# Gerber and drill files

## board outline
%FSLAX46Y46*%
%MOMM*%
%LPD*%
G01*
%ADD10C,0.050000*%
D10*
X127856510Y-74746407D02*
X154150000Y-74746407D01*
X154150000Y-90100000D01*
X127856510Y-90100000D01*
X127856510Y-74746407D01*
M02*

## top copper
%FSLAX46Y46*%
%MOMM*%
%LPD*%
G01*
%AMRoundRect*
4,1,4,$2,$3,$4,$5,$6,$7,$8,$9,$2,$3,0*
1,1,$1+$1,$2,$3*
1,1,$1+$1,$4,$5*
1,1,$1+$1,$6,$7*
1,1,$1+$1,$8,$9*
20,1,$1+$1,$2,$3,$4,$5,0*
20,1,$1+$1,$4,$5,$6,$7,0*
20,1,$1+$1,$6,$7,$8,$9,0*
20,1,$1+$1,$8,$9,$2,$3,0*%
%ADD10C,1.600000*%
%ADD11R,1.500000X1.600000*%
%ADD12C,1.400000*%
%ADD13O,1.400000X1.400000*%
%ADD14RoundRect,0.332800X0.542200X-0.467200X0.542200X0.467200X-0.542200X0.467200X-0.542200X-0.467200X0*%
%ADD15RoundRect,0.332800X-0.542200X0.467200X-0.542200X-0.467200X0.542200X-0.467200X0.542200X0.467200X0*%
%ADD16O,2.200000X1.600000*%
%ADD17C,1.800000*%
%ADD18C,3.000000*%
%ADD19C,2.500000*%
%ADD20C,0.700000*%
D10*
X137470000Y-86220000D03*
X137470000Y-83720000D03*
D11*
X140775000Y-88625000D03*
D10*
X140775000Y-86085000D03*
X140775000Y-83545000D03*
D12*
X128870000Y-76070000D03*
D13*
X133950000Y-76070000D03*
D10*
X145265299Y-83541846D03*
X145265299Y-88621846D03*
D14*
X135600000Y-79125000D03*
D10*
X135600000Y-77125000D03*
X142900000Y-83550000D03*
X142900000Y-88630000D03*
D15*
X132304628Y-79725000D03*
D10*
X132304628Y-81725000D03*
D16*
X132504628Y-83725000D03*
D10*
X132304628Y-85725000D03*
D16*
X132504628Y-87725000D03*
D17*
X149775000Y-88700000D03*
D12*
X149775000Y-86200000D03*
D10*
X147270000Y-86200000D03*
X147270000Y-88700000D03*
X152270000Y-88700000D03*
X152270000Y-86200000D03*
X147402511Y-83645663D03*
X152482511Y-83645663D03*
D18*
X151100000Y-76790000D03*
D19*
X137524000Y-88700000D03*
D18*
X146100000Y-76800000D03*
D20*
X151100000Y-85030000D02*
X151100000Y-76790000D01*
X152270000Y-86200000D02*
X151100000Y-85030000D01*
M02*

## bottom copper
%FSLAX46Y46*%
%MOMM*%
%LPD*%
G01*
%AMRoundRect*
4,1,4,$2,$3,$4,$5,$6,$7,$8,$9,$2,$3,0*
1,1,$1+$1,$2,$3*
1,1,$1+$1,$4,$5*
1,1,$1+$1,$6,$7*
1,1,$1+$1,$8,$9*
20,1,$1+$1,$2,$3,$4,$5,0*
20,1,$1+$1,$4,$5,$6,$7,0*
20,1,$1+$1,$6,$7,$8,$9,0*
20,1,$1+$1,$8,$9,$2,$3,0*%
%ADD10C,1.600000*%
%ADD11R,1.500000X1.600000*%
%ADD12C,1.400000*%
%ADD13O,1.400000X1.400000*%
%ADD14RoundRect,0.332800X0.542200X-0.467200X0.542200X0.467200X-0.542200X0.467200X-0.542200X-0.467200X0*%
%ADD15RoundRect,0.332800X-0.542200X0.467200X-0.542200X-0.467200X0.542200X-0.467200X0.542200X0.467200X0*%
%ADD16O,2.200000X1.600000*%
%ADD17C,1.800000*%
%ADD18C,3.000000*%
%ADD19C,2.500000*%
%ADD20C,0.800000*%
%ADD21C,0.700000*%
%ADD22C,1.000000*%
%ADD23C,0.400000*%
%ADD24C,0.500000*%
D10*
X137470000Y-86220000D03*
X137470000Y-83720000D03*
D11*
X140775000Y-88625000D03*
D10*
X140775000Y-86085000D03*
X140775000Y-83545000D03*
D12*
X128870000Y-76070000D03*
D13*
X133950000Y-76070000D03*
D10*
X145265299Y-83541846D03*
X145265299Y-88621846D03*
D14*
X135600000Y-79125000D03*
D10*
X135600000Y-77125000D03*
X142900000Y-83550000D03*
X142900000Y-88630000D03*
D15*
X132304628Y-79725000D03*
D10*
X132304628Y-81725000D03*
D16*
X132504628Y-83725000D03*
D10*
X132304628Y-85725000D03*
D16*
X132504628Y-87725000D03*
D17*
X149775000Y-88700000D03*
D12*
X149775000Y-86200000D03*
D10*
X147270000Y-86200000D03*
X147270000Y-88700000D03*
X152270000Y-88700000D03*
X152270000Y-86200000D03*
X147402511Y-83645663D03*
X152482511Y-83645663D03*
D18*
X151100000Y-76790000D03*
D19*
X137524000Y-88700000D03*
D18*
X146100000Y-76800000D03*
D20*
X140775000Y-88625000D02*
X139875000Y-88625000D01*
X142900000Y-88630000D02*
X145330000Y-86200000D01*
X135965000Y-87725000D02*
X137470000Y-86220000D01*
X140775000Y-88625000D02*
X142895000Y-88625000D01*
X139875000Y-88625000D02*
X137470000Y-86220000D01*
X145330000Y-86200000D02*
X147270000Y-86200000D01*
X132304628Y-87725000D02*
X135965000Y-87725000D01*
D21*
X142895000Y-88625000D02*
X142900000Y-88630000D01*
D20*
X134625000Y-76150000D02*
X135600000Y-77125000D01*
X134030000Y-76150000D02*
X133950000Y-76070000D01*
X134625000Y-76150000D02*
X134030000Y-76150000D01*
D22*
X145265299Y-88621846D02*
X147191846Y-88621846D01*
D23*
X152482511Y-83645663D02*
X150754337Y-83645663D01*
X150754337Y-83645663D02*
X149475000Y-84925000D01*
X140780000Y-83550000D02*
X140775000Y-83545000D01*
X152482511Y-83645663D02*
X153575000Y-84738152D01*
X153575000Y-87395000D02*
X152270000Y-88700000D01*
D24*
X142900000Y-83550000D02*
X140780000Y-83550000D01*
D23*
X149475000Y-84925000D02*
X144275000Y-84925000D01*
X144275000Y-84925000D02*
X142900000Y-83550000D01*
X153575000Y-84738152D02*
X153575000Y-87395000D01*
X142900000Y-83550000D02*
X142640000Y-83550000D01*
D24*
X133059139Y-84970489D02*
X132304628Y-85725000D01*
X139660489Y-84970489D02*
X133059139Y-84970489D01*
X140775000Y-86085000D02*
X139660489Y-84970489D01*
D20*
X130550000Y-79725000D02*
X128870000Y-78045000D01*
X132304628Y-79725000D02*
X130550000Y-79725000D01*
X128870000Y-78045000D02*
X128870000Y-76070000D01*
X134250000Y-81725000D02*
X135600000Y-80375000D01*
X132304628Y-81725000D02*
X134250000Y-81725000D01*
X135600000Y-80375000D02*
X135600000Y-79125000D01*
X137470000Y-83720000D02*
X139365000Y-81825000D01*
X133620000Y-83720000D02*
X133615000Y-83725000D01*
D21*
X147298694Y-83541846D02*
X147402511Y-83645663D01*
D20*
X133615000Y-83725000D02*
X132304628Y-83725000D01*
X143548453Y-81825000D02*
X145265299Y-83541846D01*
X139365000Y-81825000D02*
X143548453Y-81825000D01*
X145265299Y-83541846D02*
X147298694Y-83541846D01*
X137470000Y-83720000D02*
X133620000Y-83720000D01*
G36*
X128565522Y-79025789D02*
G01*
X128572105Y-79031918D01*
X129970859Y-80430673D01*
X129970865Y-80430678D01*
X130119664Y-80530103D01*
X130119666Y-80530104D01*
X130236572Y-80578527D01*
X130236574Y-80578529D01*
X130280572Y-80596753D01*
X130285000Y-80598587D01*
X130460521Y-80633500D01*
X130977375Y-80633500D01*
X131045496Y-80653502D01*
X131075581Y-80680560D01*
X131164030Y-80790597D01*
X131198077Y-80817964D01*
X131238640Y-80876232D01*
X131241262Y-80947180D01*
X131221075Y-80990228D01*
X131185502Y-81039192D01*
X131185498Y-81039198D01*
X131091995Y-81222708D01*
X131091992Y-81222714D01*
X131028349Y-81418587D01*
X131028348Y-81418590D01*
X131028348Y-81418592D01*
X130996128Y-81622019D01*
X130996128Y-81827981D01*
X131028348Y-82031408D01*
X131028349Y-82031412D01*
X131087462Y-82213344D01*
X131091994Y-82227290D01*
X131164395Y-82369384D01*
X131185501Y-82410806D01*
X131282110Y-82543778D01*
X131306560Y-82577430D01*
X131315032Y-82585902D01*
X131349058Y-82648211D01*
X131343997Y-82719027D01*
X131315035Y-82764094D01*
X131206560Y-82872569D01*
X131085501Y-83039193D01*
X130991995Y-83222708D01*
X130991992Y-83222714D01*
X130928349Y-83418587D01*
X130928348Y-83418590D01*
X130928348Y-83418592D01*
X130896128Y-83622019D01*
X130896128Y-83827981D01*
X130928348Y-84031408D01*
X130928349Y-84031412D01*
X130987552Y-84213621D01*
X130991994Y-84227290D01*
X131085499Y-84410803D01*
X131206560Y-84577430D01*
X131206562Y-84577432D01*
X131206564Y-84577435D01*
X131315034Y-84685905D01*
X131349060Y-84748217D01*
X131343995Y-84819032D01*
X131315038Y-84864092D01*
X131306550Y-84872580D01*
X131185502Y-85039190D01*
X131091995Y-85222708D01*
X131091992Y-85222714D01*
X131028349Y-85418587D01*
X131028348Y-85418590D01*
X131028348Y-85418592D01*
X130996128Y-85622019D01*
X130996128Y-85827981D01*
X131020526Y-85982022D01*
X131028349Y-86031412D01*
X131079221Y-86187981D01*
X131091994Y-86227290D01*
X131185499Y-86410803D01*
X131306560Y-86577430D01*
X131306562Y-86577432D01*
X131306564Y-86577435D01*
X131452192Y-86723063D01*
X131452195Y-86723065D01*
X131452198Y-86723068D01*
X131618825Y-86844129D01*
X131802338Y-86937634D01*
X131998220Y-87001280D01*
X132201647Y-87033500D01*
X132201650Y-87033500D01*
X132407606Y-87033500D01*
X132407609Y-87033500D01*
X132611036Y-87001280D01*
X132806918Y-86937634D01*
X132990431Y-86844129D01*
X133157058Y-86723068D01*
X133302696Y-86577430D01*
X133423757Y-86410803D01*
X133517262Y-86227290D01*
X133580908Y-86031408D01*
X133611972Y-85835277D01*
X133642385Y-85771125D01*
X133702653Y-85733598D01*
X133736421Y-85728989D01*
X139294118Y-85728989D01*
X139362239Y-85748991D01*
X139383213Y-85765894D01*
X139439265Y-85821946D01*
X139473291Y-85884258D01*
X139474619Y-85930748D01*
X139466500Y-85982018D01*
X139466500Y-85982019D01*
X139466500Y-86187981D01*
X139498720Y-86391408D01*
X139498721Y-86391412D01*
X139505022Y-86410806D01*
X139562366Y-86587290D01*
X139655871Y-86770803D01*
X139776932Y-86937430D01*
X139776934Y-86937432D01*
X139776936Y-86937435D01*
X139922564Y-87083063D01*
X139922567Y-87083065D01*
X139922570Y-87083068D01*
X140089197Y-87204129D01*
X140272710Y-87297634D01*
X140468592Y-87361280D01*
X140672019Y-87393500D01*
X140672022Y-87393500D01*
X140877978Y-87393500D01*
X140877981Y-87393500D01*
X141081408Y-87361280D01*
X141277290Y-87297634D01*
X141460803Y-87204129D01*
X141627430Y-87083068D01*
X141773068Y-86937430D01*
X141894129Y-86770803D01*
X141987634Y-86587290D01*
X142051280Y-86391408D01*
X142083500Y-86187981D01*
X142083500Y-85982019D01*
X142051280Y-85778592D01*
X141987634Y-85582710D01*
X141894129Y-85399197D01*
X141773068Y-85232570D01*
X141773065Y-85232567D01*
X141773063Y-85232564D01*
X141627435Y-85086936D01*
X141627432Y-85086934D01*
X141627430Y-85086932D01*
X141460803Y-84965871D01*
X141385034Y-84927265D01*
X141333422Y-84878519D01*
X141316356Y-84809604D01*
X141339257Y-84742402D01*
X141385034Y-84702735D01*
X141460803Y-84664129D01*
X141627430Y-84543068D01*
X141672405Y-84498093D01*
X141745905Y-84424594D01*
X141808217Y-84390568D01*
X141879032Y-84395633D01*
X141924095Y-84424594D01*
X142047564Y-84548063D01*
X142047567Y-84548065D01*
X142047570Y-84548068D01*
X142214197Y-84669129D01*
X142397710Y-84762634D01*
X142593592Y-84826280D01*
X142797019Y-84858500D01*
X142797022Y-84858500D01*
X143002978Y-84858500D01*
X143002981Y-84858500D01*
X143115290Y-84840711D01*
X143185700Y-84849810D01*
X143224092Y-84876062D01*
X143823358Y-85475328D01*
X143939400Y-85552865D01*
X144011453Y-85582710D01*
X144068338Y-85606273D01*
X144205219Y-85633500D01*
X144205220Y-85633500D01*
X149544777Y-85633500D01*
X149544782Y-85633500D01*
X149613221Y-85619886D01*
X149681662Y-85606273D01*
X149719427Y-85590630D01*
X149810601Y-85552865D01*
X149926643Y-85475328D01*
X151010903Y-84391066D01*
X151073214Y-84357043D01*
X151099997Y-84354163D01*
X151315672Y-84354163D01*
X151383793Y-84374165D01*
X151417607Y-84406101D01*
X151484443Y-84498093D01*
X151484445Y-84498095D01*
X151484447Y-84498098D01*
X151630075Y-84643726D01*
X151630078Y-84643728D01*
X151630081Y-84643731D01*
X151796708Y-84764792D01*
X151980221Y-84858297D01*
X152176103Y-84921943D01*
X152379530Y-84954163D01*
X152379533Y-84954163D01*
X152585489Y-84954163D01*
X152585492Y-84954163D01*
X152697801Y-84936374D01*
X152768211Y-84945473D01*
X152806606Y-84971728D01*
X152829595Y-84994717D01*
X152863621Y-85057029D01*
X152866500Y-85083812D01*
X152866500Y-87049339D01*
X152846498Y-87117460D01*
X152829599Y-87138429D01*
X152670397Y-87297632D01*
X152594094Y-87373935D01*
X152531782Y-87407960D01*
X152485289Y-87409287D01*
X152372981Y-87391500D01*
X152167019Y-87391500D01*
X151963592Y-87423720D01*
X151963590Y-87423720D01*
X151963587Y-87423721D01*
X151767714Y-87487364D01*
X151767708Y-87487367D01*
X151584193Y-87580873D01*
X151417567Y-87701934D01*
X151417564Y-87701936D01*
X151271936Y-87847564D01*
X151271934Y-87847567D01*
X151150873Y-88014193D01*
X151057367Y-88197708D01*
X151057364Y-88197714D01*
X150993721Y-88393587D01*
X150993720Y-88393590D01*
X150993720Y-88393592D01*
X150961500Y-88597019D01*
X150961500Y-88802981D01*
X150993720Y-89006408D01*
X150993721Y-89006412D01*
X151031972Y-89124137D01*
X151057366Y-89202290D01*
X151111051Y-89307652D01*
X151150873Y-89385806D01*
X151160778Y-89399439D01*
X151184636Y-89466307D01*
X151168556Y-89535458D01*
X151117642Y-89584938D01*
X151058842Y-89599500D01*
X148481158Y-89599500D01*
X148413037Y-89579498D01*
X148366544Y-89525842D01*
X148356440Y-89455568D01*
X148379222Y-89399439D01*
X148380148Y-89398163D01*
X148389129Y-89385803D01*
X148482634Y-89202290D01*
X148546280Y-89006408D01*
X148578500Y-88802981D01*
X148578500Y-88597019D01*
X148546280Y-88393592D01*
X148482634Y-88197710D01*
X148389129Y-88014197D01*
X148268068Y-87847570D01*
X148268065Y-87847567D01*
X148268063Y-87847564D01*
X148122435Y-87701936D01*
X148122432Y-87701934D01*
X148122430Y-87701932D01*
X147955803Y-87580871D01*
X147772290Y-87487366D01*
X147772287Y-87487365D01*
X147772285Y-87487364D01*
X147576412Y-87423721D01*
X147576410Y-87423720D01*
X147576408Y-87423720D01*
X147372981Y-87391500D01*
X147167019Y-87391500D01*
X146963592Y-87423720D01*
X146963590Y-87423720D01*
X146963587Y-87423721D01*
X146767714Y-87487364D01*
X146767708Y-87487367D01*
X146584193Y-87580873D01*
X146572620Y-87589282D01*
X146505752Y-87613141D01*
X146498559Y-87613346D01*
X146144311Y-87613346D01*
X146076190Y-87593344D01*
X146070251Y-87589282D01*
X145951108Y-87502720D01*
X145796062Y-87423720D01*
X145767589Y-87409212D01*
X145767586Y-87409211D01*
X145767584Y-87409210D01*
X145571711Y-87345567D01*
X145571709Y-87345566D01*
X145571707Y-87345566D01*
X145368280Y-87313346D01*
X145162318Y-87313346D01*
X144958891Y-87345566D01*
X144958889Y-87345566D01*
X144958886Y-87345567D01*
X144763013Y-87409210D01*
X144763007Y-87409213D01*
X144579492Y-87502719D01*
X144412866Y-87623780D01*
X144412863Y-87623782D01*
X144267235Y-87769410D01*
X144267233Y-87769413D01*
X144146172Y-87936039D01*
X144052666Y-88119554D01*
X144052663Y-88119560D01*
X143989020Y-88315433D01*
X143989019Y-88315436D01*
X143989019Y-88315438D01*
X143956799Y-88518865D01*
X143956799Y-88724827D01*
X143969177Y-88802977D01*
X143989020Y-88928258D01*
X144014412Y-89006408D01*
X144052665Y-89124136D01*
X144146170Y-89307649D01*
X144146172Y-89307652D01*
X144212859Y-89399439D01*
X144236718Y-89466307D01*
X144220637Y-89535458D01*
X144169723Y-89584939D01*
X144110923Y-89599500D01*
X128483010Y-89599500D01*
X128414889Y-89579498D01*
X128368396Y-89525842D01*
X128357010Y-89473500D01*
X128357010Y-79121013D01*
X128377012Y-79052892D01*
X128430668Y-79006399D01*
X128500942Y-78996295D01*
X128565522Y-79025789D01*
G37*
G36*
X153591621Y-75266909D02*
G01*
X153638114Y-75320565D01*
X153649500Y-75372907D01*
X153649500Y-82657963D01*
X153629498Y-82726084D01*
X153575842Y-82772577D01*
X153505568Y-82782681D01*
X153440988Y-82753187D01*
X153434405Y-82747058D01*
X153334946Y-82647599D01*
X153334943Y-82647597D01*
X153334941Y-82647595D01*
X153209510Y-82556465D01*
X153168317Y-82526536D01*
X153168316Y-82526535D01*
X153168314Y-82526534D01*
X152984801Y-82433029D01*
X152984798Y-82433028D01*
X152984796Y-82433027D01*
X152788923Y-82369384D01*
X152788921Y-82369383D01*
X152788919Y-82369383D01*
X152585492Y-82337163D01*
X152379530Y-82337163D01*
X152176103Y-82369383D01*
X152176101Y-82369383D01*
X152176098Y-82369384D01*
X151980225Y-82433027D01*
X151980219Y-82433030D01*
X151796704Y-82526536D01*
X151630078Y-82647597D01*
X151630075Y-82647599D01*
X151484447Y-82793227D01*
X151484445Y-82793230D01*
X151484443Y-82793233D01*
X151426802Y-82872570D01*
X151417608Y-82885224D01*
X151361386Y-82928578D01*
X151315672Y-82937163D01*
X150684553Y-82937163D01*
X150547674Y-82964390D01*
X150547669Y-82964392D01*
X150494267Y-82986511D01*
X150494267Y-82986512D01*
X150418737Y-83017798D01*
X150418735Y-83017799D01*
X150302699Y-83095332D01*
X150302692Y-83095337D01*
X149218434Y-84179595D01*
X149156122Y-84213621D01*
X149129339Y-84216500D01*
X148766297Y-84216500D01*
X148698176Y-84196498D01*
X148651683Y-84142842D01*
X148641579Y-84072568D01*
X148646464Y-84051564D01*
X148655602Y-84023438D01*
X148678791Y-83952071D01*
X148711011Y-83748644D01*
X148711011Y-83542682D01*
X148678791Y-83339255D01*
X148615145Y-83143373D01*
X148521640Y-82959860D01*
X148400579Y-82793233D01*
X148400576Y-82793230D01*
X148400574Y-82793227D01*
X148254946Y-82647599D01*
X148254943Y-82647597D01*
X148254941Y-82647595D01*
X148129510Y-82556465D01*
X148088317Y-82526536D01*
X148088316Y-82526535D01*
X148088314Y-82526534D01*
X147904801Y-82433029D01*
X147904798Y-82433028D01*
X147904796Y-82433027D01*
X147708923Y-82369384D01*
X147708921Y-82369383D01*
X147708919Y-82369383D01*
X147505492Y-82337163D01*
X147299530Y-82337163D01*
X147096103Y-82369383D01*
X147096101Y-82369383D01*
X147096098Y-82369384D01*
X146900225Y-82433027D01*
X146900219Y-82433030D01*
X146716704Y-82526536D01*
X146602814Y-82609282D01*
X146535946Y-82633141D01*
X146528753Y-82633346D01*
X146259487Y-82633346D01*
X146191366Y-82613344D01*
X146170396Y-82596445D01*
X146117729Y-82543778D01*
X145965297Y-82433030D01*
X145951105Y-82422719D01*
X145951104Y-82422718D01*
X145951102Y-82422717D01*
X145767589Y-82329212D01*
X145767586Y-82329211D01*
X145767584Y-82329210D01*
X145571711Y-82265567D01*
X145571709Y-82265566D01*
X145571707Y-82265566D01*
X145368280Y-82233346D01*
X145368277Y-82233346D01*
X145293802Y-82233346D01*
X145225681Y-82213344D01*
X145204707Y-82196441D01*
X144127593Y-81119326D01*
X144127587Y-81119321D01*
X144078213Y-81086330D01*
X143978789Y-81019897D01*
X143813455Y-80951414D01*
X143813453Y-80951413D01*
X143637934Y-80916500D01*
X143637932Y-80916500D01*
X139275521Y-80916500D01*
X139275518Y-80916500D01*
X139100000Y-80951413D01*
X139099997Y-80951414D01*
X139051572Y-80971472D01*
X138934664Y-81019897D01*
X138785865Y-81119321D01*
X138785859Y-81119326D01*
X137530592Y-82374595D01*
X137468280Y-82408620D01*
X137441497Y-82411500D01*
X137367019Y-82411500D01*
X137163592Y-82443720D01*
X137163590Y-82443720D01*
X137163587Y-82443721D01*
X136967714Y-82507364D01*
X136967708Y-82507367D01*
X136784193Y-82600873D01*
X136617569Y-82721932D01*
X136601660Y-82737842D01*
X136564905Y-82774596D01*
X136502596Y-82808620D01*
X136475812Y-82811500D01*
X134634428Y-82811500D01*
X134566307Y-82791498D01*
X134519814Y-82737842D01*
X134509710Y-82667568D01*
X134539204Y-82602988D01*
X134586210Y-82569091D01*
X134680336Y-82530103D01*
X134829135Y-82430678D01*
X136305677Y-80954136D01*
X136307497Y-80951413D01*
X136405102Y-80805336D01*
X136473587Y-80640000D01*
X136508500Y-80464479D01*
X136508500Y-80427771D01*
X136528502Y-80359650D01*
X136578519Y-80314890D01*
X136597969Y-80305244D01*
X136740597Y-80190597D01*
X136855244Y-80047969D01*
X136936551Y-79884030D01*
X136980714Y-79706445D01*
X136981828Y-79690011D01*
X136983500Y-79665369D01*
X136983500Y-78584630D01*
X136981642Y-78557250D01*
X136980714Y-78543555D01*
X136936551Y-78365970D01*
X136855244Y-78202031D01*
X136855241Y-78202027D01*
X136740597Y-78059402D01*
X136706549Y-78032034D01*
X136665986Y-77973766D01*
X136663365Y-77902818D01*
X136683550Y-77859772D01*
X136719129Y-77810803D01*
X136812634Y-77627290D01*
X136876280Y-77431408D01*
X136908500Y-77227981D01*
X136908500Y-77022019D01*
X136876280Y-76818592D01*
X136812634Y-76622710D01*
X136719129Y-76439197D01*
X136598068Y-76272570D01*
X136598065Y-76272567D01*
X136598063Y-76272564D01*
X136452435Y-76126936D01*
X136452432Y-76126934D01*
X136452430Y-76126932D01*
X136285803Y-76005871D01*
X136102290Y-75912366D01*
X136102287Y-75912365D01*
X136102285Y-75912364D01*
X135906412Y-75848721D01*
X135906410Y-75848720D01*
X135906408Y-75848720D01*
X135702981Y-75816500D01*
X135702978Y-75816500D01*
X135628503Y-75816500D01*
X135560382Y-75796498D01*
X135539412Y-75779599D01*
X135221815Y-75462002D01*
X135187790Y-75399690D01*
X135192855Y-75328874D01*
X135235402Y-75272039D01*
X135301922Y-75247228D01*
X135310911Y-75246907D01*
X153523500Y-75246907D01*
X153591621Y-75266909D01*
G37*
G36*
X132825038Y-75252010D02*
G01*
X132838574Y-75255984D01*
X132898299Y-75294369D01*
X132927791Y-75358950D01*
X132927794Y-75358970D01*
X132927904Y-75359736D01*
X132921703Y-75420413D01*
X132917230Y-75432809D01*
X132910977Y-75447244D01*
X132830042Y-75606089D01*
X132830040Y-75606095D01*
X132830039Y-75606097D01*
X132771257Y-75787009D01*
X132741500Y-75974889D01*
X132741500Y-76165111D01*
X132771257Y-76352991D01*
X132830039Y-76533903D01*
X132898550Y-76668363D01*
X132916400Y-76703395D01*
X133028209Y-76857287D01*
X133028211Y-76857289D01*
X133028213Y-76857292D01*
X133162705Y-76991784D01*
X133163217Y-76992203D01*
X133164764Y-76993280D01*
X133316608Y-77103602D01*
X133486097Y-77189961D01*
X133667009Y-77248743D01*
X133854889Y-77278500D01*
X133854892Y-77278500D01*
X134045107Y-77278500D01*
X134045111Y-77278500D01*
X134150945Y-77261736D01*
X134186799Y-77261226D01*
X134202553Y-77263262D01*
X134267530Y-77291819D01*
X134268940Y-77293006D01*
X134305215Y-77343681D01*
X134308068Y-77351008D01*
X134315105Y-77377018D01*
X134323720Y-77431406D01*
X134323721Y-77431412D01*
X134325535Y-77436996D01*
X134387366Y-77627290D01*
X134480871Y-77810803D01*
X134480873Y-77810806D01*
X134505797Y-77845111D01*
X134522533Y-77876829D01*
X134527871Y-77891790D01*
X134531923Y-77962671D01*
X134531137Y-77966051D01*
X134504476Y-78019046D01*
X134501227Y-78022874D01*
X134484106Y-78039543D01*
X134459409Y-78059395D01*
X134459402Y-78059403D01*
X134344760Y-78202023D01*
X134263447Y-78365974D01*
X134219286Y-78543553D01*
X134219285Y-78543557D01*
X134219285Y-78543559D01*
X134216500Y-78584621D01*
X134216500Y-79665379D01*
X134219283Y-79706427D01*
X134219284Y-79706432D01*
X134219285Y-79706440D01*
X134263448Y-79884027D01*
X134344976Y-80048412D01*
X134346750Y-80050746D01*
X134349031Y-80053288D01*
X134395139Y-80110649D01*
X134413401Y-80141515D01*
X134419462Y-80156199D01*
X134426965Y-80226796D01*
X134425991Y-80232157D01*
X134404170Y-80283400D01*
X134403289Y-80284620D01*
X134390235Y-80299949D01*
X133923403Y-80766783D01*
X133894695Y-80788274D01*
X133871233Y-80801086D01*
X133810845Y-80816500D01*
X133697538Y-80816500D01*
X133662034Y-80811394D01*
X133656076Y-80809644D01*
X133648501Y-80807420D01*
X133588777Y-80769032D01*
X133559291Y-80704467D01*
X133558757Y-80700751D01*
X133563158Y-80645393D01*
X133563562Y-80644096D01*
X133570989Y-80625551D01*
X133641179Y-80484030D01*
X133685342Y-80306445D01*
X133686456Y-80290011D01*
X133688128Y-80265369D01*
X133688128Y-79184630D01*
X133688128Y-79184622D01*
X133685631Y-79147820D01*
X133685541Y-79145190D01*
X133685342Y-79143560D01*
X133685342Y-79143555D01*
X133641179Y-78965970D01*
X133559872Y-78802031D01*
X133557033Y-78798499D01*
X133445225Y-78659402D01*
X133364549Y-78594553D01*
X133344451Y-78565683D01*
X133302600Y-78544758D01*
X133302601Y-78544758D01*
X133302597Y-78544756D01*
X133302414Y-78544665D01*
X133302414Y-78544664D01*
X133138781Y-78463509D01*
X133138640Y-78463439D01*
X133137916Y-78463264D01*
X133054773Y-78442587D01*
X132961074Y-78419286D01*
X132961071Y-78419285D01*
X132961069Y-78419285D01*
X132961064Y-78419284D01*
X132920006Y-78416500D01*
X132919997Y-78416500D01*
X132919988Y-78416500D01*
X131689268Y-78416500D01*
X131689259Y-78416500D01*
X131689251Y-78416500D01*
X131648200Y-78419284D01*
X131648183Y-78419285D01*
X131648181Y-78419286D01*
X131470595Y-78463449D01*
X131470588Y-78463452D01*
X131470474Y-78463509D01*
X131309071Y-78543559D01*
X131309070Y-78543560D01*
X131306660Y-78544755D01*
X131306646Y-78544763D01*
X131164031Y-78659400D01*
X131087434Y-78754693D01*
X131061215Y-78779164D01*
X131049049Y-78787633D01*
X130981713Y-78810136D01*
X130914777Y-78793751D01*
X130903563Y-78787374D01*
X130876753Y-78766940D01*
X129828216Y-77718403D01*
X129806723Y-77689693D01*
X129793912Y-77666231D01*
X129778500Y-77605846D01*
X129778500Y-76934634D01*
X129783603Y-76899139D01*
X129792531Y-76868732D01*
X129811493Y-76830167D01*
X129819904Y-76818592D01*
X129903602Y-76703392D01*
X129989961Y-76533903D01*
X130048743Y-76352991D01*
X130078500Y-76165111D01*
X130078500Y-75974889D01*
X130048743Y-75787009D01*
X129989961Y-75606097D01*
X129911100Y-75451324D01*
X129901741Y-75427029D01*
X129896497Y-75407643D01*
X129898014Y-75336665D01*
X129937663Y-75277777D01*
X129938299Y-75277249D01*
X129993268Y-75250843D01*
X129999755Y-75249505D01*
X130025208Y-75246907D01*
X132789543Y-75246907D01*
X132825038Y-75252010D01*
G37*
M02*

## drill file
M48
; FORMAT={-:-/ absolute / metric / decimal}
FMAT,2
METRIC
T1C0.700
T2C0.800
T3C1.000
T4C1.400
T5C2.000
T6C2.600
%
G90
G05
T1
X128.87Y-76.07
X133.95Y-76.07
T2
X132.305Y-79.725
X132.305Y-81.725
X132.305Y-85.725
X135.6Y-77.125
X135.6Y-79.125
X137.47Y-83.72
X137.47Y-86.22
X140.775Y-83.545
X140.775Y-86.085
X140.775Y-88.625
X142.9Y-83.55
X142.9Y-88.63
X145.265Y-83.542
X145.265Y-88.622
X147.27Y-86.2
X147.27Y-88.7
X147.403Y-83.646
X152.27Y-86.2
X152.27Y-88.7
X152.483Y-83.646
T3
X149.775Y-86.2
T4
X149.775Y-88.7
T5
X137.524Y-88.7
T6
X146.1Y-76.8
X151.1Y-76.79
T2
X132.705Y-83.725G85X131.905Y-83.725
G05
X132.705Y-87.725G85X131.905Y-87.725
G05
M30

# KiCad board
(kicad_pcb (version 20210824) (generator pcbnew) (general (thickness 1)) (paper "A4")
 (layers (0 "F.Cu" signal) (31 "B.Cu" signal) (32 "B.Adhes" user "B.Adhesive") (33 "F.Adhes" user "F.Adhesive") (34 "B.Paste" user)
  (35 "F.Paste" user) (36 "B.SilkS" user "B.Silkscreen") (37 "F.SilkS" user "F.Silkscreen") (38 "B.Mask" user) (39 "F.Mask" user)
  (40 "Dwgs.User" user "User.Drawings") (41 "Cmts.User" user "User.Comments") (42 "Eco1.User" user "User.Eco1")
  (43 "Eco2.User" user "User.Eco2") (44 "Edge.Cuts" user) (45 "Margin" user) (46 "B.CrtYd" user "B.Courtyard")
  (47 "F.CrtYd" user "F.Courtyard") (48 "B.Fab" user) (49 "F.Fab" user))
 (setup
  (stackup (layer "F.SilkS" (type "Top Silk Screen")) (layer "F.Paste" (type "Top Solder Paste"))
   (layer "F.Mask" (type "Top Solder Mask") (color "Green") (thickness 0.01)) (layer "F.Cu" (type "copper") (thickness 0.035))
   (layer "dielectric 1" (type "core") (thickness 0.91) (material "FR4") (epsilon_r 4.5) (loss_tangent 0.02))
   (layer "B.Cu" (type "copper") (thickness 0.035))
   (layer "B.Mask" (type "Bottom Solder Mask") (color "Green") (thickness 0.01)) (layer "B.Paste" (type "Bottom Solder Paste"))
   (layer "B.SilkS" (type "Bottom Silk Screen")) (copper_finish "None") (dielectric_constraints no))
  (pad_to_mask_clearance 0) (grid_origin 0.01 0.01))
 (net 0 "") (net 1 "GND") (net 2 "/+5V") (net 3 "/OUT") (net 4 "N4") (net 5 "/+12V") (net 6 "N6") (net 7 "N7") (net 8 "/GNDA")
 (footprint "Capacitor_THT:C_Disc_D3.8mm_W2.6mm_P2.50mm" (layer "F.Cu") (at 137.47 86.22 90)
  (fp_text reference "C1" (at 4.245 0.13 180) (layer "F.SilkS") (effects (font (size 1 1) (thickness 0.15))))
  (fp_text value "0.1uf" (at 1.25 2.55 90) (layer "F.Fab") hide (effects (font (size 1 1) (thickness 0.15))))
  (pad "1" thru_hole circle locked (at 0 0 90) (size 1.6 1.6) (drill 0.8) (layers *.Cu *.Mask) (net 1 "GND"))
  (pad "2" thru_hole circle locked (at 2.5 0 90) (size 1.6 1.6) (drill 0.8) (layers *.Cu *.Mask) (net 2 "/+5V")))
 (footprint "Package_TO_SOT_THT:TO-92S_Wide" (layer "F.Cu") (at 140.775 88.625 90)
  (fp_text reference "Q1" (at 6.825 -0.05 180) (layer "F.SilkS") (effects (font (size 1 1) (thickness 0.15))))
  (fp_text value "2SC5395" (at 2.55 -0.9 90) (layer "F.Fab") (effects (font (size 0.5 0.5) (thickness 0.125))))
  (pad "1" thru_hole rect locked (at 0 0 90) (size 1.6 1.5) (drill 0.8) (layers *.Cu *.Mask) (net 1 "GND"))
  (pad "2" thru_hole circle locked (at 2.54 0 90) (size 1.6 1.6) (drill 0.8) (layers *.Cu *.Mask) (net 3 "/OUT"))
  (pad "3" thru_hole circle locked (at 5.08 0 90) (size 1.6 1.6) (drill 0.8) (layers *.Cu *.Mask) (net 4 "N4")))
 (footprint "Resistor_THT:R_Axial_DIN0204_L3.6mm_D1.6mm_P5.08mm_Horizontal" (layer "F.Cu") (at 128.87 76.07)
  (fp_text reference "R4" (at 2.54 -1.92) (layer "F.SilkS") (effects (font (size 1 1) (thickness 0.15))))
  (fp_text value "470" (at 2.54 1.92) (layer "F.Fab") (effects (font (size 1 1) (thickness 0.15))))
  (pad "1" thru_hole circle locked (at 0 0) (size 1.4 1.4) (drill 0.7) (layers *.Cu *.Mask) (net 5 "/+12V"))
  (pad "2" thru_hole oval locked (at 5.08 0) (size 1.4 1.4) (drill 0.7) (layers *.Cu *.Mask) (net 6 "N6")))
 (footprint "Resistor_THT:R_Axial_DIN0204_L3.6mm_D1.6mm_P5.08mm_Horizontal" (layer "F.Cu") (at 145.265299 83.541846 -90)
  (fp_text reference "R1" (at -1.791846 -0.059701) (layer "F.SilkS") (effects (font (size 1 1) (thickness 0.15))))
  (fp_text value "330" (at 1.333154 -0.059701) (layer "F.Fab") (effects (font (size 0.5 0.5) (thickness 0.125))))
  (pad "1" thru_hole circle locked (at 0 0 270) (size 1.6 1.6) (drill 0.8) (layers *.Cu *.Mask) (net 2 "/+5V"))
  (pad "2" thru_hole circle locked (at 5.08 0 270) (size 1.6 1.6) (drill 0.8) (layers *.Cu *.Mask) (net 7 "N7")))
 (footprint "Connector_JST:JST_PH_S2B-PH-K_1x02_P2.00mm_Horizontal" (layer "F.Cu") (at 135.6 79.125 90)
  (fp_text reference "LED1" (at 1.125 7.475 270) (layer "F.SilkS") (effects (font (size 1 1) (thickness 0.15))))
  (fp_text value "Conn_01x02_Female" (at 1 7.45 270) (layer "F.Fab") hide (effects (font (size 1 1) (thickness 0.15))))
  (pad "1" thru_hole roundrect locked (at 0 0 90) (size 1.6 1.75) (drill 0.8) (layers *.Cu *.Mask) (roundrect_rratio 0.208) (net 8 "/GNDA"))
  (pad "2" thru_hole circle locked (at 2 0 90) (size 1.6 1.6) (drill 0.8) (layers *.Cu *.Mask) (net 6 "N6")))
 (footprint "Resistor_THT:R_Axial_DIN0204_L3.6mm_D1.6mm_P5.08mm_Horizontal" (layer "F.Cu") (at 142.9 83.55 -90)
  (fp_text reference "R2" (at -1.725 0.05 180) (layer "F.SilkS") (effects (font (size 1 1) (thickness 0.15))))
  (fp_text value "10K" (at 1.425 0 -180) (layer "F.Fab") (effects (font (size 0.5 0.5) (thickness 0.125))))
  (pad "1" thru_hole circle locked (at 0 0 270) (size 1.6 1.6) (drill 0.8) (layers *.Cu *.Mask) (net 4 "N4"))
  (pad "2" thru_hole circle locked (at 5.08 0 270) (size 1.6 1.6) (drill 0.8) (layers *.Cu *.Mask) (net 1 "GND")))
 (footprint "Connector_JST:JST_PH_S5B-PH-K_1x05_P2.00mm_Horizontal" (layer "F.Cu") (at 132.304628 79.725 -90)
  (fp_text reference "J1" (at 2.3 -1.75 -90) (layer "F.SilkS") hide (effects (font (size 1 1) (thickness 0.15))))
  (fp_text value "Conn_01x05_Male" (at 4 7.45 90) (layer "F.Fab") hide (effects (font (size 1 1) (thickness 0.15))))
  (pad "1" thru_hole roundrect locked (at 0 0 270) (size 1.6 1.75) (drill 0.8) (layers *.Cu *.Mask) (roundrect_rratio 0.208) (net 5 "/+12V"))
  (pad "2" thru_hole circle locked (at 2 0 270) (size 1.6 1.6) (drill 0.8) (layers *.Cu *.Mask) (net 8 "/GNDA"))
  (pad "3" thru_hole oval locked (at 4 0 270) (size 1.6 2.2) (drill oval 0.8 1.6 (offset 0 -0.2)) (layers *.Cu *.Mask) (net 2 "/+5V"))
  (pad "4" thru_hole circle locked (at 6 0 270) (size 1.6 1.6) (drill 0.8) (layers *.Cu *.Mask) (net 3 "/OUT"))
  (pad "5" thru_hole oval locked (at 8 0 270) (size 1.6 2.2) (drill oval 0.8 1.6 (offset 0 -0.2)) (layers *.Cu *.Mask) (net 1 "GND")))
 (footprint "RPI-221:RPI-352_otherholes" (layer "F.Cu") (at 149.775 86.18)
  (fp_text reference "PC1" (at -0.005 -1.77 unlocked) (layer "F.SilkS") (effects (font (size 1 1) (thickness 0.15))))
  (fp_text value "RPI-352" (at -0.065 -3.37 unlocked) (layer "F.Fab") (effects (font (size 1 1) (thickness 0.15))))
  (pad "" thru_hole circle (at 0 2.52) (size 1.8 1.8) (drill 1.4) (layers *.Cu *.Mask) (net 1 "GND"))
  (pad "" thru_hole circle (at 0 0.02) (size 1.4 1.4) (drill 1) (layers *.Cu *.Mask) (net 1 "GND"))
  (pad "1" thru_hole circle locked (at -2.505 0.02) (size 1.6 1.6) (drill 0.8) (layers *.Cu *.Mask) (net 1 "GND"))
  (pad "2" thru_hole circle locked (at -2.505 2.52) (size 1.6 1.6) (drill 0.8) (layers *.Cu *.Mask) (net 7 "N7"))
  (pad "3" thru_hole circle locked (at 2.495 2.52) (size 1.6 1.6) (drill 0.8) (layers *.Cu *.Mask) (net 4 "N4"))
  (pad "4" thru_hole circle locked (at 2.495 0.02) (size 1.6 1.6) (drill 0.8) (layers *.Cu *.Mask) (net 1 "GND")))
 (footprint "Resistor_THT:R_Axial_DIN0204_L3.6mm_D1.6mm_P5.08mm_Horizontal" (layer "F.Cu") (at 147.402511 83.645663)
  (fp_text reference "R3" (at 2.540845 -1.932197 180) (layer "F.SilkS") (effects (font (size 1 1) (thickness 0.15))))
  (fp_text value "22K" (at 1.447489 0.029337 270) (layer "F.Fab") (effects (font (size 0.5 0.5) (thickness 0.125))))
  (pad "1" thru_hole circle locked (at 0 0) (size 1.6 1.6) (drill 0.8) (layers *.Cu *.Mask) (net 2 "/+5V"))
  (pad "2" thru_hole circle locked (at 5.08 0) (size 1.6 1.6) (drill 0.8) (layers *.Cu *.Mask) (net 4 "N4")))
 (gr_rect (start 127.85651 74.746407) (end 154.15 90.1) (layer "Edge.Cuts") (width 0.05) (fill none))
 (segment (start 151.1 85.03) (end 151.1 76.79) (width 0.7) (layer "F.Cu") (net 1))
 (segment (start 152.27 86.2) (end 151.1 85.03) (width 0.7) (layer "F.Cu") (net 1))
 (via (at 151.1 76.79) (size 3) (drill 2.6) (layers "F.Cu" "B.Cu") (free) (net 1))
 (via (at 137.524 88.7) (size 2.5) (drill 2) (layers "F.Cu" "B.Cu") (free) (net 1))
 (via (at 146.1 76.8) (size 3) (drill 2.6) (layers "F.Cu" "B.Cu") (free) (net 1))
 (segment (start 140.775 88.625) (end 139.875 88.625) (width 0.8) (layer "B.Cu") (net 1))
 (segment (start 142.9 88.63) (end 145.33 86.2) (width 0.8) (layer "B.Cu") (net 1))
 (segment (start 135.965 87.725) (end 137.47 86.22) (width 0.8) (layer "B.Cu") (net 1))
 (segment (start 140.775 88.625) (end 142.895 88.625) (width 0.8) (layer "B.Cu") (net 1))
 (segment (start 139.875 88.625) (end 137.47 86.22) (width 0.8) (layer "B.Cu") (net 1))
 (segment (start 145.33 86.2) (end 147.27 86.2) (width 0.8) (layer "B.Cu") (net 1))
 (segment (start 132.304628 87.725) (end 135.965 87.725) (width 0.8) (layer "B.Cu") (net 1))
 (segment (start 142.895 88.625) (end 142.9 88.63) (width 0.7) (layer "B.Cu") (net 1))
 (segment (start 134.625 76.15) (end 135.6 77.125) (width 0.8) (layer "B.Cu") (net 6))
 (segment (start 134.03 76.15) (end 133.95 76.07) (width 0.8) (layer "B.Cu") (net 6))
 (segment (start 134.625 76.15) (end 134.03 76.15) (width 0.8) (layer "B.Cu") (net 6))
 (segment (start 145.265299 88.621846) (end 147.191846 88.621846) (width 1) (layer "B.Cu") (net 7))
 (segment (start 152.482511 83.645663) (end 150.754337 83.645663) (width 0.4) (layer "B.Cu") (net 4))
 (segment (start 150.754337 83.645663) (end 149.475 84.925) (width 0.4) (layer "B.Cu") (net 4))
 (segment (start 140.78 83.55) (end 140.775 83.545) (width 0.4) (layer "B.Cu") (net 4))
 (segment (start 152.482511 83.645663) (end 153.575 84.738152) (width 0.4) (layer "B.Cu") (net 4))
 (segment (start 153.575 87.395) (end 152.27 88.7) (width 0.4) (layer "B.Cu") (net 4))
 (segment (start 142.9 83.55) (end 140.78 83.55) (width 0.5) (layer "B.Cu") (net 4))
 (segment (start 149.475 84.925) (end 144.275 84.925) (width 0.4) (layer "B.Cu") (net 4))
 (segment (start 144.275 84.925) (end 142.9 83.55) (width 0.4) (layer "B.Cu") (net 4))
 (segment (start 153.575 84.738152) (end 153.575 87.395) (width 0.4) (layer "B.Cu") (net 4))
 (segment (start 142.9 83.55) (end 142.64 83.55) (width 0.4) (layer "B.Cu") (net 4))
 (segment (start 133.059139 84.970489) (end 132.304628 85.725) (width 0.5) (layer "B.Cu") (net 3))
 (segment (start 139.660489 84.970489) (end 133.059139 84.970489) (width 0.5) (layer "B.Cu") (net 3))
 (segment (start 140.775 86.085) (end 139.660489 84.970489) (width 0.5) (layer "B.Cu") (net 3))
 (segment (start 130.55 79.725) (end 128.87 78.045) (width 0.8) (layer "B.Cu") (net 5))
 (segment (start 132.304628 79.725) (end 130.55 79.725) (width 0.8) (layer "B.Cu") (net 5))
 (segment (start 128.87 78.045) (end 128.87 76.07) (width 0.8) (layer "B.Cu") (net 5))
 (segment (start 134.25 81.725) (end 135.6 80.375) (width 0.8) (layer "B.Cu") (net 8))
 (segment (start 132.304628 81.725) (end 134.25 81.725) (width 0.8) (layer "B.Cu") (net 8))
 (segment (start 135.6 80.375) (end 135.6 79.125) (width 0.8) (layer "B.Cu") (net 8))
 (segment (start 137.47 83.72) (end 139.365 81.825) (width 0.8) (layer "B.Cu") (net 2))
 (segment (start 133.62 83.72) (end 133.615 83.725) (width 0.8) (layer "B.Cu") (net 2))
 (segment (start 147.298694 83.541846) (end 147.402511 83.645663) (width 0.7) (layer "B.Cu") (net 2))
 (segment (start 133.615 83.725) (end 132.304628 83.725) (width 0.8) (layer "B.Cu") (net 2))
 (segment (start 143.548453 81.825) (end 145.265299 83.541846) (width 0.8) (layer "B.Cu") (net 2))
 (segment (start 139.365 81.825) (end 143.548453 81.825) (width 0.8) (layer "B.Cu") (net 2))
 (segment (start 145.265299 83.541846) (end 147.298694 83.541846) (width 0.8) (layer "B.Cu") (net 2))
 (segment (start 137.47 83.72) (end 133.62 83.72) (width 0.8) (layer "B.Cu") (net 2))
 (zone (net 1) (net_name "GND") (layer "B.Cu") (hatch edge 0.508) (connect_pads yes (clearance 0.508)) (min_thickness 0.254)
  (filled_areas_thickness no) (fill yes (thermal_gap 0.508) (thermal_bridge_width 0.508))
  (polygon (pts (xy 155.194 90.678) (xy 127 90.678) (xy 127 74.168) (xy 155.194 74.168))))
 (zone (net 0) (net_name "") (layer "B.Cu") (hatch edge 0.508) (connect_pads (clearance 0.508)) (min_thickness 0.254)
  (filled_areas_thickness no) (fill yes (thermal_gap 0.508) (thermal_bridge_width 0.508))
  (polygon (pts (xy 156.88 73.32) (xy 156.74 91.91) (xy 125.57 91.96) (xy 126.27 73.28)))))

